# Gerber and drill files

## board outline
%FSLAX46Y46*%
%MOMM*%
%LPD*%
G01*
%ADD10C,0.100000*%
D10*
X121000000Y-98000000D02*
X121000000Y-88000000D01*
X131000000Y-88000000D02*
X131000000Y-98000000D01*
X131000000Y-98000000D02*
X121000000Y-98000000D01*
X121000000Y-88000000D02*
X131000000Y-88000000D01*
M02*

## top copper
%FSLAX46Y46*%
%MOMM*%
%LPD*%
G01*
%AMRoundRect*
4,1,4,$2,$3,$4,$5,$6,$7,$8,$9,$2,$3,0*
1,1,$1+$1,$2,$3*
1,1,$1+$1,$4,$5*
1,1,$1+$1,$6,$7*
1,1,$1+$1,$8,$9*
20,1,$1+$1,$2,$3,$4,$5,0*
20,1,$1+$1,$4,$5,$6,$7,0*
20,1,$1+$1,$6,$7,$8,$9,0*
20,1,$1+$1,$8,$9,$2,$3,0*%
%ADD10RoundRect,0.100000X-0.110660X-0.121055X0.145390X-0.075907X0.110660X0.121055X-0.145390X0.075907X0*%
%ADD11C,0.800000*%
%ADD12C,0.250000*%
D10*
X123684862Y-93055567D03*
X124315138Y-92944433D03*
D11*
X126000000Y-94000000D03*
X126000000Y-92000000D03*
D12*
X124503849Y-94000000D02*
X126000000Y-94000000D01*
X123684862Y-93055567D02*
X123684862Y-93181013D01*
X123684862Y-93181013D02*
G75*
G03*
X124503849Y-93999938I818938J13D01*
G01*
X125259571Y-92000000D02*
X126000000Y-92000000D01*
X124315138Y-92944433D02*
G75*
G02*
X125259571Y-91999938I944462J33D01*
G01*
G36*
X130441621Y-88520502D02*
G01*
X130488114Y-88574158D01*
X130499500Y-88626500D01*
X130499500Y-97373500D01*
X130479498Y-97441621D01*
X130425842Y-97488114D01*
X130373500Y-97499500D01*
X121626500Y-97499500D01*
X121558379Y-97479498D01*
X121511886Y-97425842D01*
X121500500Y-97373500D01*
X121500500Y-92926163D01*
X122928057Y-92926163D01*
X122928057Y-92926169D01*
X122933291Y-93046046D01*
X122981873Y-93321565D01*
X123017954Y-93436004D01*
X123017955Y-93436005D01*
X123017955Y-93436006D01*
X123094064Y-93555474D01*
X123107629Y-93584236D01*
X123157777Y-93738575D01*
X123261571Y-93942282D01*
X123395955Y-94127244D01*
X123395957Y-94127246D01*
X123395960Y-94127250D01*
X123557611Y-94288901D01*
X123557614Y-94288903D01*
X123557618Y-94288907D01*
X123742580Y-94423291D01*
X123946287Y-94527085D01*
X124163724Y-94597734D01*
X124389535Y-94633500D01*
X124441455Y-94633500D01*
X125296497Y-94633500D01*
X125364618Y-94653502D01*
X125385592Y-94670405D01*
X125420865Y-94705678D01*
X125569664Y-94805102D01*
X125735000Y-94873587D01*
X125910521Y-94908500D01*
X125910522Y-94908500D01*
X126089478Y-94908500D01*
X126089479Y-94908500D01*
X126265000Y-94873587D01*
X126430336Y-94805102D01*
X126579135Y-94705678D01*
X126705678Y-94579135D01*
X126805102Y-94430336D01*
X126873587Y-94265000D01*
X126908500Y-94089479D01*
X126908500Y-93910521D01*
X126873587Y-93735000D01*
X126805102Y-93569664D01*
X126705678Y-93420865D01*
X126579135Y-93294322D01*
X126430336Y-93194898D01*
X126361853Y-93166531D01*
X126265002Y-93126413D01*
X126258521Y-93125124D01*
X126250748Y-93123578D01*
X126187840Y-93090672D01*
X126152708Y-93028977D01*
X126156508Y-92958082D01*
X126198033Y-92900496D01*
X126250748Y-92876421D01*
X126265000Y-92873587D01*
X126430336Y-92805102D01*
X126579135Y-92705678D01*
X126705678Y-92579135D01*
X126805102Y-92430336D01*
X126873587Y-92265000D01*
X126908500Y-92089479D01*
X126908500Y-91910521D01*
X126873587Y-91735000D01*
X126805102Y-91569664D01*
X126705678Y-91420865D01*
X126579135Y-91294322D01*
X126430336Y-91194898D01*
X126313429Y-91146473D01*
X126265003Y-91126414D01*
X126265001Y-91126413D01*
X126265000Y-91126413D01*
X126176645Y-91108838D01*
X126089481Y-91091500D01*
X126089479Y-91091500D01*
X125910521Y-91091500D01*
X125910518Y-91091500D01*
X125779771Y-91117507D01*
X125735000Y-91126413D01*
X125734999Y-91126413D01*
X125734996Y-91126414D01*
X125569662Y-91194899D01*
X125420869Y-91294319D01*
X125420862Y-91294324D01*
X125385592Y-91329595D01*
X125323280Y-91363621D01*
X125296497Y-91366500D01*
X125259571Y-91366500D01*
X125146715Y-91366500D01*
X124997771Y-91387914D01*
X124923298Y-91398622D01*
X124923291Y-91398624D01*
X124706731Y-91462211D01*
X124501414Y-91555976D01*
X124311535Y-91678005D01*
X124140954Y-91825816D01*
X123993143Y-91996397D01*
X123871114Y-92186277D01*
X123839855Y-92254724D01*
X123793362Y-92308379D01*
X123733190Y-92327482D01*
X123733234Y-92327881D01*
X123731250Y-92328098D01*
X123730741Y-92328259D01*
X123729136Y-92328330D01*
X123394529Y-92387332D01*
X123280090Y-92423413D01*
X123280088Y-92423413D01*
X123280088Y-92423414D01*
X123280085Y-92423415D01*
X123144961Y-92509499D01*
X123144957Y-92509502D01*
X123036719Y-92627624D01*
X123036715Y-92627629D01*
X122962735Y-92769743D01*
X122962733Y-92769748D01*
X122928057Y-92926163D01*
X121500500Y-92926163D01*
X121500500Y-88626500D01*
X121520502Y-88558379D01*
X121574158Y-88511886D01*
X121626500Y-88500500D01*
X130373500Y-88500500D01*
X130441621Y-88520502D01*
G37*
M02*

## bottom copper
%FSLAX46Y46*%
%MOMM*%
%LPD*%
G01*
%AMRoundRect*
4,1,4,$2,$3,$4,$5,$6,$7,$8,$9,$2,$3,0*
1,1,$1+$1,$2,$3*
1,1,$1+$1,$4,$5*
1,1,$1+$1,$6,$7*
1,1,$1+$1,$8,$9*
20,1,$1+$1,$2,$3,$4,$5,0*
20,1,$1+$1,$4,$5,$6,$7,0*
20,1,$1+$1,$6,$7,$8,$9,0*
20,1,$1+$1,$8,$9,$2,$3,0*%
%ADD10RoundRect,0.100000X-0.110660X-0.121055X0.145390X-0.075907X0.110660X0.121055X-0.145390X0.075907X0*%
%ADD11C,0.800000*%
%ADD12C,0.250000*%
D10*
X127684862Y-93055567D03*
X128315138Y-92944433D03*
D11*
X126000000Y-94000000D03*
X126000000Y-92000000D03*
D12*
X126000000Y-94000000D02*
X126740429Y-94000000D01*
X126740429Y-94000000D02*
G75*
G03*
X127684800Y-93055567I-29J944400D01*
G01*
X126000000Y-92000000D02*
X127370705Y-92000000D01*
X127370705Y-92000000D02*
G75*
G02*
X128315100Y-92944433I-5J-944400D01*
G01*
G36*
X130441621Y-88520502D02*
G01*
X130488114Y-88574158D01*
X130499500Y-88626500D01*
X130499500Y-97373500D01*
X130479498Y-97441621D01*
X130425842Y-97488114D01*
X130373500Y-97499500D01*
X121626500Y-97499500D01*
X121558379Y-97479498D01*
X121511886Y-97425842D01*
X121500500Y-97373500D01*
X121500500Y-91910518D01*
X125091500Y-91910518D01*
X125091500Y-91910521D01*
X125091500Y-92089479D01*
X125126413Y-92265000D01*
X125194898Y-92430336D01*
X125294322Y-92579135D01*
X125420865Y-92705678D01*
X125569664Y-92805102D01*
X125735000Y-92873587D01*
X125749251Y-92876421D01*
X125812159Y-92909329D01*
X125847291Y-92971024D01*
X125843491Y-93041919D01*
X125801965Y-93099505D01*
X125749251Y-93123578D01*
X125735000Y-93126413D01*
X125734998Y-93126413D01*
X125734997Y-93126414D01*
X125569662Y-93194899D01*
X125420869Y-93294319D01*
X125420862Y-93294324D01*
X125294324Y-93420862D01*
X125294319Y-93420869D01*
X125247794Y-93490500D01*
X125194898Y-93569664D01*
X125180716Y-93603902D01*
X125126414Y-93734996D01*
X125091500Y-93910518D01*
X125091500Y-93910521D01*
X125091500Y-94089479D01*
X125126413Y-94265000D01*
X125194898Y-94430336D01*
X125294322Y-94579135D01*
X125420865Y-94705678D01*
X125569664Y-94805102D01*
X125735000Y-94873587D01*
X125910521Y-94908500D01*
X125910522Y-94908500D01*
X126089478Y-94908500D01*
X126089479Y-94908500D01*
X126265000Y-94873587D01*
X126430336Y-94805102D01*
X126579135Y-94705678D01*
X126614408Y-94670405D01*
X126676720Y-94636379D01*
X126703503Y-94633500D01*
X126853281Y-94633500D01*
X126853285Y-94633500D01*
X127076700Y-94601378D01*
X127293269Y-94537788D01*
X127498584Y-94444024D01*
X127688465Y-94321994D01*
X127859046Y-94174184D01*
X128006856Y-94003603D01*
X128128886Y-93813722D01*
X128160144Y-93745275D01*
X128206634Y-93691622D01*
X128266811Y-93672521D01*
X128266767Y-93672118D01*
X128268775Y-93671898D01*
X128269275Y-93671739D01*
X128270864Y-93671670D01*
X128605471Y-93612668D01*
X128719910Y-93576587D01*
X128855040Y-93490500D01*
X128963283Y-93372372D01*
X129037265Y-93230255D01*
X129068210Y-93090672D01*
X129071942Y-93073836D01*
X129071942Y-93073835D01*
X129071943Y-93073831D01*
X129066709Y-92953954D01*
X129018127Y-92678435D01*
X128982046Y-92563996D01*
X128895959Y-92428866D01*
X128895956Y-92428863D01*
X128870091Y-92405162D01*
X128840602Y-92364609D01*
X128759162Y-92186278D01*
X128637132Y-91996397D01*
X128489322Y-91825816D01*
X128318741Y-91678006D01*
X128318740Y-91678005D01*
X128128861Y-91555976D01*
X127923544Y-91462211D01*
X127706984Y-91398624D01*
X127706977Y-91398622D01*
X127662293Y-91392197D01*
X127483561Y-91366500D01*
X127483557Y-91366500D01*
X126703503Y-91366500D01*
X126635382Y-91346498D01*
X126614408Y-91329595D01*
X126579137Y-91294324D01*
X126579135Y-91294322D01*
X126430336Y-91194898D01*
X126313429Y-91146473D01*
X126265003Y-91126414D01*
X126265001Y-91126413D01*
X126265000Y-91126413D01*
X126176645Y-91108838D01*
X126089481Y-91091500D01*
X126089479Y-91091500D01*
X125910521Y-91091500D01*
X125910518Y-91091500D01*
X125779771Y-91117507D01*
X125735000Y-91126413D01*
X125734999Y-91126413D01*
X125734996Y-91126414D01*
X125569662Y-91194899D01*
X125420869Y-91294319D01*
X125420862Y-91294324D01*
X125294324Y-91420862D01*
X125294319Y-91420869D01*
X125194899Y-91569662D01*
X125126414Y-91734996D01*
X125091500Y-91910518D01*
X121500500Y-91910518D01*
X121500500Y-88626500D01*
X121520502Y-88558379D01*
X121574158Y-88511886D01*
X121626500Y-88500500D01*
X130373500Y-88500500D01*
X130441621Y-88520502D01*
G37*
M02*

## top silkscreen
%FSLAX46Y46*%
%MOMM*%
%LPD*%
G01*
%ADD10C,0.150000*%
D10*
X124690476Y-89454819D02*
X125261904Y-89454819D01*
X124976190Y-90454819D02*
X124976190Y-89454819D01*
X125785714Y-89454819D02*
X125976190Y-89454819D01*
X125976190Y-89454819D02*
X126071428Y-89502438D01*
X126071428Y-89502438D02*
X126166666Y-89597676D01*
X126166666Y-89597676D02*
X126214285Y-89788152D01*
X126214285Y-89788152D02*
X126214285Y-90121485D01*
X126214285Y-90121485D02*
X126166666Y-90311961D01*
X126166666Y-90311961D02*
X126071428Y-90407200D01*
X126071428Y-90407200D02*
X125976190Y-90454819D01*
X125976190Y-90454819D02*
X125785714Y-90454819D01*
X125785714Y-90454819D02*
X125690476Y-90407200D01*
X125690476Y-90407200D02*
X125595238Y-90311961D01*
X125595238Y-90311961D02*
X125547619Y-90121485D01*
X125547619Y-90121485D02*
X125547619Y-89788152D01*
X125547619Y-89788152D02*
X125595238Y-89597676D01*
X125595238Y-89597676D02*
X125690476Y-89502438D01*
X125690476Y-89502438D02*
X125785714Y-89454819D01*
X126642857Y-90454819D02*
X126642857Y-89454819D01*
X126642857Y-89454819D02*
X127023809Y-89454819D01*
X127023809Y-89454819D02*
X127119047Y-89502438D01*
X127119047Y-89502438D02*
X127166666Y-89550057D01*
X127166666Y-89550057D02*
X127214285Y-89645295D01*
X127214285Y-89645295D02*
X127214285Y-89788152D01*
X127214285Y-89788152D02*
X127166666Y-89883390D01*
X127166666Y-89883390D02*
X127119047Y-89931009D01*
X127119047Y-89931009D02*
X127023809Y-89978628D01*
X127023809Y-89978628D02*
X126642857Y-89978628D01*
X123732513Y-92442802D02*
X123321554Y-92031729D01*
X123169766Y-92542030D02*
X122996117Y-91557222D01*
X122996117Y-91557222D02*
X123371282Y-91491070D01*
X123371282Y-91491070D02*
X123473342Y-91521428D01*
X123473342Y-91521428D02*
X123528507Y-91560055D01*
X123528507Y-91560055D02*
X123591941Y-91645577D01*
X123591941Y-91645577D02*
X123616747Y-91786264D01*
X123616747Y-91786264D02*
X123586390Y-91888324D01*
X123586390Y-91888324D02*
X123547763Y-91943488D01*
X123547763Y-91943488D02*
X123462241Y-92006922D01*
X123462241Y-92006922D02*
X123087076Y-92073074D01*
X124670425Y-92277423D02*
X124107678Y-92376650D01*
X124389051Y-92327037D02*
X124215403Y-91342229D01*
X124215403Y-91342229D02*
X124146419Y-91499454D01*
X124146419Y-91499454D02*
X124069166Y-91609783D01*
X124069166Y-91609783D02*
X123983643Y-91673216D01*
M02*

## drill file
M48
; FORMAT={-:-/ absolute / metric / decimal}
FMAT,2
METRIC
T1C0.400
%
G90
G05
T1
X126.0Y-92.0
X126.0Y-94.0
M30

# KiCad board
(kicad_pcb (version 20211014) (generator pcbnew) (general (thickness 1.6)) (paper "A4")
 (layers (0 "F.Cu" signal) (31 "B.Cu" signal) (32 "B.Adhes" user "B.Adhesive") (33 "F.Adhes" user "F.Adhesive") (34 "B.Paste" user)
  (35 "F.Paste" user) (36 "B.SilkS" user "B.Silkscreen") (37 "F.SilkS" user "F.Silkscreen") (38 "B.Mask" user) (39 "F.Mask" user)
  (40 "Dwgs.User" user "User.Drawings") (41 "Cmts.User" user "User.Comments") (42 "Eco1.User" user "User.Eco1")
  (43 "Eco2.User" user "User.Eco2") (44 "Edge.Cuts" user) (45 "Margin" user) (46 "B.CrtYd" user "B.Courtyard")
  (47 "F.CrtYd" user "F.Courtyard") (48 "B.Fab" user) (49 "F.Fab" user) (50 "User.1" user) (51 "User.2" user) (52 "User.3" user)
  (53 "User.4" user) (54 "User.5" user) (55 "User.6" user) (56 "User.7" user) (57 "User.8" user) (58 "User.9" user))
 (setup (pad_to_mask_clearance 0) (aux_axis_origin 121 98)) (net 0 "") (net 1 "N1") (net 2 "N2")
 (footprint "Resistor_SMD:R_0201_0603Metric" (layer "F.Cu") (at 124 93 10)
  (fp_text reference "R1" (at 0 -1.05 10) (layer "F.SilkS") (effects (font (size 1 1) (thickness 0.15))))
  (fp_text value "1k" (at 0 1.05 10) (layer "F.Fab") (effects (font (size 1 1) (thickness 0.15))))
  (pad "" smd roundrect (at 0.345 0 10) (size 0.318 0.36) (layers "F.Paste") (roundrect_rratio 0.25))
  (pad "" smd roundrect (at -0.345 0 10) (size 0.318 0.36) (layers "F.Paste") (roundrect_rratio 0.25))
  (pad "1" smd roundrect (at -0.32 0 10) (size 0.46 0.4) (layers "F.Cu" "F.Mask") (roundrect_rratio 0.25) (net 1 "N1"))
  (pad "2" smd roundrect (at 0.32 0 10) (size 0.46 0.4) (layers "F.Cu" "F.Mask") (roundrect_rratio 0.25) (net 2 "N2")))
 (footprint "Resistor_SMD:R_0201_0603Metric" (layer "B.Cu") (at 128 93 10)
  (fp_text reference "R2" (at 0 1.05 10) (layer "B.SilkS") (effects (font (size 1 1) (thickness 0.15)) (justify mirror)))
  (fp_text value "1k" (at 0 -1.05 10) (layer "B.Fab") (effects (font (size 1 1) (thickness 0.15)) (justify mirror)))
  (pad "" smd roundrect (at 0.345 0 10) (size 0.318 0.36) (layers "B.Paste") (roundrect_rratio 0.25))
  (pad "" smd roundrect (at -0.345 0 10) (size 0.318 0.36) (layers "B.Paste") (roundrect_rratio 0.25))
  (pad "1" smd roundrect (at -0.32 0 10) (size 0.46 0.4) (layers "B.Cu" "B.Mask") (roundrect_rratio 0.25) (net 1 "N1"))
  (pad "2" smd roundrect (at 0.32 0 10) (size 0.46 0.4) (layers "B.Cu" "B.Mask") (roundrect_rratio 0.25) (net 2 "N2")))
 (gr_line (start 121 98) (end 121 88) (layer "Edge.Cuts") (width 0.1))
 (gr_line (start 131 88) (end 131 98) (layer "Edge.Cuts") (width 0.1))
 (gr_line (start 131 98) (end 121 98) (layer "Edge.Cuts") (width 0.1))
 (gr_line (start 121 88) (end 131 88) (layer "Edge.Cuts") (width 0.1))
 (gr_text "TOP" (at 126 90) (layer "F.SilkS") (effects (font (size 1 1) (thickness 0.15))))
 (segment (start 124.503849 94) (end 126 94) (width 0.25) (layer "F.Cu") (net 1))
 (segment (start 123.684862 93.055567) (end 123.684862 93.181013) (width 0.25) (layer "F.Cu") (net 1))
 (via (at 126 94) (size 0.8) (drill 0.4) (layers "F.Cu" "B.Cu") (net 1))
 (arc (start 123.684862 93.181013) (mid 123.924738 93.760124) (end 124.503849 94) (width 0.25) (layer "F.Cu") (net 1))
 (segment (start 126 94) (end 126.740429 94) (width 0.25) (layer "B.Cu") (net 1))
 (arc (start 126.740429 94) (mid 127.408244 93.723382) (end 127.684862 93.055567) (width 0.25) (layer "B.Cu") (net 1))
 (segment (start 125.259571 92) (end 126 92) (width 0.25) (layer "F.Cu") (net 2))
 (via (at 126 92) (size 0.8) (drill 0.4) (layers "F.Cu" "B.Cu") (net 2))
 (arc (start 124.315138 92.944433) (mid 124.591756 92.276618) (end 125.259571 92) (width 0.25) (layer "F.Cu") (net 2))
 (segment (start 126 92) (end 127.370705 92) (width 0.25) (layer "B.Cu") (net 2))
 (arc (start 127.370705 92) (mid 128.03852 92.276618) (end 128.315138 92.944433) (width 0.25) (layer "B.Cu") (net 2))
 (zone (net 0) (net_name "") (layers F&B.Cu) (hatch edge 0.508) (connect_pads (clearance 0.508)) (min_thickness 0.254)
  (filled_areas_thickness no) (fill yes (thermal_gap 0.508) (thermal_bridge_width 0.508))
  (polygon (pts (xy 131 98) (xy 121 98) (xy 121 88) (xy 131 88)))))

